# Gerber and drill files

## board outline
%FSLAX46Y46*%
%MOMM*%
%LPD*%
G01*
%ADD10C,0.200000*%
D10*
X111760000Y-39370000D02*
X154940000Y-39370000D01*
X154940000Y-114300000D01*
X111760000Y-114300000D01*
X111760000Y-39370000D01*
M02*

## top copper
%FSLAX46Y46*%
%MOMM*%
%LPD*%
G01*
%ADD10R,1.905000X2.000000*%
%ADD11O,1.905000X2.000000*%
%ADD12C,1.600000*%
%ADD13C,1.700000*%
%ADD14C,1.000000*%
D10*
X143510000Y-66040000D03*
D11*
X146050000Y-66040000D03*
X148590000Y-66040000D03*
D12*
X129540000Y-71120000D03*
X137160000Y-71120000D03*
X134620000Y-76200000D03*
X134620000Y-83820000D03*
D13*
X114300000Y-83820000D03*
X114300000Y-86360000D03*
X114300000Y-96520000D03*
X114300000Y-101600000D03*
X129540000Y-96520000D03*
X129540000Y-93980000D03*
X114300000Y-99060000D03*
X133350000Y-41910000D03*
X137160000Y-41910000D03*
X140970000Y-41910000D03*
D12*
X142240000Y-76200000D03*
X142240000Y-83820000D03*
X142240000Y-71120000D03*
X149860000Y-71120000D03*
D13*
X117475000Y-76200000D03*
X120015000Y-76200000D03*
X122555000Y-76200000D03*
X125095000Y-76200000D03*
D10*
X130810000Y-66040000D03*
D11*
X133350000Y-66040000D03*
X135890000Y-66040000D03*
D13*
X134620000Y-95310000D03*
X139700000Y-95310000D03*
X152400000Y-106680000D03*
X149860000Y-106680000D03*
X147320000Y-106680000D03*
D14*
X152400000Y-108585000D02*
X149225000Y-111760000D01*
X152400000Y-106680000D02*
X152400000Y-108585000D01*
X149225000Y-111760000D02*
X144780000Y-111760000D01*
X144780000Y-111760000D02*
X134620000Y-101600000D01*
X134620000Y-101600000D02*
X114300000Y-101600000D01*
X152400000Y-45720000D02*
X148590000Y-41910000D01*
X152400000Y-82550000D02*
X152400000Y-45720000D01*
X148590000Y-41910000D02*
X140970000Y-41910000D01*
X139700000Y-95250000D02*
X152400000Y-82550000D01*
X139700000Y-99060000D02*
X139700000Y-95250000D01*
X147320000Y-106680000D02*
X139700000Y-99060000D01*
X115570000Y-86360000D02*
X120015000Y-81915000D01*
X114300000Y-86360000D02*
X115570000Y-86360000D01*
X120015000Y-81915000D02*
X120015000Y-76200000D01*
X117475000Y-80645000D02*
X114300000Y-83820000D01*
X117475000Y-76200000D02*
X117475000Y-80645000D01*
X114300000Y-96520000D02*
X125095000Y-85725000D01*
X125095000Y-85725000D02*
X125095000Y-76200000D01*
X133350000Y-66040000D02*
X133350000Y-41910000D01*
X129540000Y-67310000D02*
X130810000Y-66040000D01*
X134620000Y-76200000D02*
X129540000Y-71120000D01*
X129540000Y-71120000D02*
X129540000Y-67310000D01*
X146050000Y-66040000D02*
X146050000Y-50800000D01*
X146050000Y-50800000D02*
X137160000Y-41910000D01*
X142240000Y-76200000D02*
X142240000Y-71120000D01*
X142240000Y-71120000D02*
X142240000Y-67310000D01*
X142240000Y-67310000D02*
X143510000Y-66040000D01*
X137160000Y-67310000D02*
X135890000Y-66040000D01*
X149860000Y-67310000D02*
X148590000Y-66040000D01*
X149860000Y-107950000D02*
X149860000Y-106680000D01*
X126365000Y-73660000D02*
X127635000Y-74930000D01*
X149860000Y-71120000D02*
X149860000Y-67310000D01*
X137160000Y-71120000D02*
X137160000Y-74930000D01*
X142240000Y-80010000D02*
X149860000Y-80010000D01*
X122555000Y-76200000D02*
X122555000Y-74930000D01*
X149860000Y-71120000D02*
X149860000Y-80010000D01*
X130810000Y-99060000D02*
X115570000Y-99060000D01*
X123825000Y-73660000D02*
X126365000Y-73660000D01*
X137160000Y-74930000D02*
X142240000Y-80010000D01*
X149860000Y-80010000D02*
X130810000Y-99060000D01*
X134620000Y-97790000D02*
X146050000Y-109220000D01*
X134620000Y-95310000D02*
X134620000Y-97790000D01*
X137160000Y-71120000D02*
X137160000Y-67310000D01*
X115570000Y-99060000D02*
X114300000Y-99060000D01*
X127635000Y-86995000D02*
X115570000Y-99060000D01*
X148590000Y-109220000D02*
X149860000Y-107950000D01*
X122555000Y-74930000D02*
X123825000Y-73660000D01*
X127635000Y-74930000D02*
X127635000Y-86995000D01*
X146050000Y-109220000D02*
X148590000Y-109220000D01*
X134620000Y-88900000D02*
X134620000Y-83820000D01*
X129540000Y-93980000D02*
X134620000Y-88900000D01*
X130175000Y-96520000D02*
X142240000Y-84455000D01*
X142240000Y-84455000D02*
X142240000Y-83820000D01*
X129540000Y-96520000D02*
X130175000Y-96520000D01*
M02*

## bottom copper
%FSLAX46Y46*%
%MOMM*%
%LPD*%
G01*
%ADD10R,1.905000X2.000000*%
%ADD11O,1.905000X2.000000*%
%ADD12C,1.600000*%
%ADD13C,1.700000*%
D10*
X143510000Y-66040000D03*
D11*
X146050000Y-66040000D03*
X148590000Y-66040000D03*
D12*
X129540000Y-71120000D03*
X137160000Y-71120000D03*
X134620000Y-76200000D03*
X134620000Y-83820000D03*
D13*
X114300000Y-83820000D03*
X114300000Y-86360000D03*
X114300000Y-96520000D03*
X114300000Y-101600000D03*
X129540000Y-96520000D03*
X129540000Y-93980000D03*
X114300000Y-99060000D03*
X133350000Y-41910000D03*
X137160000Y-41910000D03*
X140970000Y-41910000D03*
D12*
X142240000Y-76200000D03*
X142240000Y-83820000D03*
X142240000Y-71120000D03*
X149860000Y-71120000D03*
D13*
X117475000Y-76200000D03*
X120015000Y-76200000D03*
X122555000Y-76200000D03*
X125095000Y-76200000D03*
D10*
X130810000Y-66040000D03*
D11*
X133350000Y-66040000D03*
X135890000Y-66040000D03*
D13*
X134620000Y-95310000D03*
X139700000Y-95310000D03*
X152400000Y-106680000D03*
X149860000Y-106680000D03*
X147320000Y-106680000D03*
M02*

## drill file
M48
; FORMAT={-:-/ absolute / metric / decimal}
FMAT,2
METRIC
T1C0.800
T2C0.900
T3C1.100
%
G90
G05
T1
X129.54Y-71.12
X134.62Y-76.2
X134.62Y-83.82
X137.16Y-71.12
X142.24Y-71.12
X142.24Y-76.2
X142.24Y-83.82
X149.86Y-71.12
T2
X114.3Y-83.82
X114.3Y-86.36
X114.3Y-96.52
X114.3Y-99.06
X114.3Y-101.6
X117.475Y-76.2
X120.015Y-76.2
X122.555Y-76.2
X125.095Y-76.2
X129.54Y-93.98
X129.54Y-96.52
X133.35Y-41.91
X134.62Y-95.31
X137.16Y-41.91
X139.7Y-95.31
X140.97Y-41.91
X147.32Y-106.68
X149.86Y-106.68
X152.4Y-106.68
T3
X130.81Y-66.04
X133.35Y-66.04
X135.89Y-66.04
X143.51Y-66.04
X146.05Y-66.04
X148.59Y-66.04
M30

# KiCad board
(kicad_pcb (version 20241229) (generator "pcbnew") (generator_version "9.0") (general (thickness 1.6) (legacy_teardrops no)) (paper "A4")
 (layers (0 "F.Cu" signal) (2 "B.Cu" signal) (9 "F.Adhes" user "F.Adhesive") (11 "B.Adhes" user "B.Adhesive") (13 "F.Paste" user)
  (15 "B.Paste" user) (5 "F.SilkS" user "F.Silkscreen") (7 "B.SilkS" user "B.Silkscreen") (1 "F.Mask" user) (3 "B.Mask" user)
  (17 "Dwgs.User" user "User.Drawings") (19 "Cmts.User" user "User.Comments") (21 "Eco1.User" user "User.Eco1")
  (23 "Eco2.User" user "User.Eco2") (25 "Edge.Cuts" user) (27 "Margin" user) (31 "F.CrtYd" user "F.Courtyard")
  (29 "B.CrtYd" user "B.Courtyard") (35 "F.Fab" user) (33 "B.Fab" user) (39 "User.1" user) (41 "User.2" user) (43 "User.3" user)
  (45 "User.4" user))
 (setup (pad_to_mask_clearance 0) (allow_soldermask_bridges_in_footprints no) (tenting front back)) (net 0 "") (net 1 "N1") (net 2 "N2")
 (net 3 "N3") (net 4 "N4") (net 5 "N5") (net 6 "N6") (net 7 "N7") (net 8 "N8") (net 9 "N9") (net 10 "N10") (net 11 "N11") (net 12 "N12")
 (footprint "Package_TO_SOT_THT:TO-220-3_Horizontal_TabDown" (layer "F.Cu") (at 143.51 66.04)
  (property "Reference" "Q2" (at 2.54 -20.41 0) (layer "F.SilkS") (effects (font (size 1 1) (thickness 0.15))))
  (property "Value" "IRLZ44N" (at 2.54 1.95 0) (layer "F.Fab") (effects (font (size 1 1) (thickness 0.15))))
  (pad "1" thru_hole rect (at 0 0) (size 1.905 2) (drill 1.1) (layers "*.Cu" "*.Mask") (remove_unused_layers no) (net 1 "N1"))
  (pad "2" thru_hole oval (at 2.54 0) (size 1.905 2) (drill 1.1) (layers "*.Cu" "*.Mask") (remove_unused_layers no) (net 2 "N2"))
  (pad "3" thru_hole oval (at 5.08 0) (size 1.905 2) (drill 1.1) (layers "*.Cu" "*.Mask") (remove_unused_layers no) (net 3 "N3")))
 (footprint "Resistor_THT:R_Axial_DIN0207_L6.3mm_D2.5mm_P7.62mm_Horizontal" (layer "F.Cu") (at 129.54 71.12)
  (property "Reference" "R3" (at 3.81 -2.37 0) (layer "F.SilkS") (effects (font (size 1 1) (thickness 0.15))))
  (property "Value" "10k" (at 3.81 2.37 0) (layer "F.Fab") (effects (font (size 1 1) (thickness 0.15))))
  (pad "1" thru_hole circle (at 0 0) (size 1.6 1.6) (drill 0.8) (layers "*.Cu" "*.Mask") (remove_unused_layers no) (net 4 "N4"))
  (pad "2" thru_hole circle (at 7.62 0) (size 1.6 1.6) (drill 0.8) (layers "*.Cu" "*.Mask") (remove_unused_layers no) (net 3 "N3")))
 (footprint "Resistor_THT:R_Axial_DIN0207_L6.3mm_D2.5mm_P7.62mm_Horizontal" (layer "F.Cu") (at 134.62 76.2 -90)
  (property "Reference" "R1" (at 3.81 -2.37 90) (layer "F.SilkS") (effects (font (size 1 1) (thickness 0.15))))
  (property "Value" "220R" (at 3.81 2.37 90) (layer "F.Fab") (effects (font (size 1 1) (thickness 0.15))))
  (pad "1" thru_hole circle (at 0 0 270) (size 1.6 1.6) (drill 0.8) (layers "*.Cu" "*.Mask") (remove_unused_layers no) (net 4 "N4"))
  (pad "2" thru_hole circle (at 7.62 0 270) (size 1.6 1.6) (drill 0.8) (layers "*.Cu" "*.Mask") (remove_unused_layers no) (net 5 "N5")))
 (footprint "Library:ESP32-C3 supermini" (layer "F.Cu") (at 121.92 91.44)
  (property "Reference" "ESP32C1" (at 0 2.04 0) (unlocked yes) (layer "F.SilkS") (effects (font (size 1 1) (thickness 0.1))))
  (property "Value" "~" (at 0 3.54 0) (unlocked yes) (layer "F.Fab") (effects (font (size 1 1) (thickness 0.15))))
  (pad "0" thru_hole circle (at -7.62 -7.62) (size 1.7 1.7) (drill 0.9) (layers "*.Cu" "*.Mask") (remove_unused_layers yes)
   (keep_end_layers yes) (zone_layer_connections) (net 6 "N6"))
  (pad "1" thru_hole circle (at -7.62 -5.08) (size 1.7 1.7) (drill 0.9) (layers "*.Cu" "*.Mask") (remove_unused_layers yes)
   (keep_end_layers yes) (zone_layer_connections) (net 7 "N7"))
  (pad "3.3V" thru_hole circle (at -7.62 5.08) (size 1.7 1.7) (drill 0.9) (layers "*.Cu" "*.Mask") (remove_unused_layers yes)
   (keep_end_layers yes) (zone_layer_connections) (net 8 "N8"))
  (pad "5V" thru_hole circle (at -7.62 10.16) (size 1.7 1.7) (drill 0.9) (layers "*.Cu" "*.Mask") (remove_unused_layers yes)
   (keep_end_layers yes) (zone_layer_connections) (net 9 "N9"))
  (pad "7" thru_hole circle (at 7.62 5.08) (size 1.7 1.7) (drill 0.9) (layers "*.Cu" "*.Mask") (remove_unused_layers yes)
   (keep_end_layers yes) (zone_layer_connections) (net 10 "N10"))
  (pad "8" thru_hole circle (at 7.62 2.54) (size 1.7 1.7) (drill 0.9) (layers "*.Cu" "*.Mask") (remove_unused_layers yes)
   (keep_end_layers yes) (zone_layer_connections) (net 5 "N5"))
  (pad "GND" thru_hole circle (at -7.62 7.62) (size 1.7 1.7) (drill 0.9) (layers "*.Cu" "*.Mask") (remove_unused_layers yes)
   (keep_end_layers yes) (zone_layer_connections) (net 3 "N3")))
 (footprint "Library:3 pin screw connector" (layer "F.Cu") (at 137.16 41.91)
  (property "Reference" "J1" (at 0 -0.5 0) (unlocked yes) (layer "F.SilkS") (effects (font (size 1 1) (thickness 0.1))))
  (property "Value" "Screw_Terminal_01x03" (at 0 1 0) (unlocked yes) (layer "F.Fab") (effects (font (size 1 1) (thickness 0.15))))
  (pad "1" thru_hole circle (at -3.81 0) (size 1.7 1.7) (drill 0.9) (layers "*.Cu" "*.Mask") (remove_unused_layers yes)
   (keep_end_layers yes) (zone_layer_connections) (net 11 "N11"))
  (pad "2" thru_hole circle (at 0 0) (size 1.7 1.7) (drill 0.9) (layers "*.Cu" "*.Mask") (remove_unused_layers yes) (keep_end_layers yes)
   (zone_layer_connections) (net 2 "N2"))
  (pad "3" thru_hole circle (at 3.81 0) (size 1.7 1.7) (drill 0.9) (layers "*.Cu" "*.Mask") (remove_unused_layers yes) (keep_end_layers yes)
   (zone_layer_connections) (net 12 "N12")))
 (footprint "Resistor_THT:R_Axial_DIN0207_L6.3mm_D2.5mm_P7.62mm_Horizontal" (layer "F.Cu") (at 142.24 76.2 -90)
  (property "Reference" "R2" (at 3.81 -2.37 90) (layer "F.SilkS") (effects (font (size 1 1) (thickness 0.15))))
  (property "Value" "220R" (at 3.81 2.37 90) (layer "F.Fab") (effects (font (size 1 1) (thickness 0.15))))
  (pad "1" thru_hole circle (at 0 0 270) (size 1.6 1.6) (drill 0.8) (layers "*.Cu" "*.Mask") (remove_unused_layers no) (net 1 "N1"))
  (pad "2" thru_hole circle (at 7.62 0 270) (size 1.6 1.6) (drill 0.8) (layers "*.Cu" "*.Mask") (remove_unused_layers no) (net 10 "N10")))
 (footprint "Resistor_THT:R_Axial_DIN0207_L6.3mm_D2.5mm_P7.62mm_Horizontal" (layer "F.Cu") (at 142.24 71.12)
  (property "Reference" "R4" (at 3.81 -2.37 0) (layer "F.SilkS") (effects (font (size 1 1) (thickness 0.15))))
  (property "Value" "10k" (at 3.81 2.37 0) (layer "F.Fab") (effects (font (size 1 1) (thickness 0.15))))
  (pad "1" thru_hole circle (at 0 0) (size 1.6 1.6) (drill 0.8) (layers "*.Cu" "*.Mask") (remove_unused_layers no) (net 1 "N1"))
  (pad "2" thru_hole circle (at 7.62 0) (size 1.6 1.6) (drill 0.8) (layers "*.Cu" "*.Mask") (remove_unused_layers no) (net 3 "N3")))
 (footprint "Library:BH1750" (layer "F.Cu") (at 120.015 68.072)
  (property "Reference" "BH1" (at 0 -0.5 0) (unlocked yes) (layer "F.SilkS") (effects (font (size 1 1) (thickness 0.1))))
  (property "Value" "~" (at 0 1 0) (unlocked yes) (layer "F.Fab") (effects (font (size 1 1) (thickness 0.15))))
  (pad "1" thru_hole circle (at -2.54 8.128 90) (size 1.7 1.7) (drill 0.9) (layers "*.Cu" "*.Mask") (remove_unused_layers yes)
   (keep_end_layers yes) (zone_layer_connections) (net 6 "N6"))
  (pad "2" thru_hole circle (at 0 8.128 90) (size 1.7 1.7) (drill 0.9) (layers "*.Cu" "*.Mask") (remove_unused_layers yes)
   (keep_end_layers yes) (zone_layer_connections) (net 7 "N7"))
  (pad "3" thru_hole circle (at 2.54 8.128 90) (size 1.7 1.7) (drill 0.9) (layers "*.Cu" "*.Mask") (remove_unused_layers yes)
   (keep_end_layers yes) (zone_layer_connections) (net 3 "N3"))
  (pad "4" thru_hole circle (at 5.08 8.128 90) (size 1.7 1.7) (drill 0.9) (layers "*.Cu" "*.Mask") (remove_unused_layers yes)
   (keep_end_layers yes) (zone_layer_connections) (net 8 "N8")))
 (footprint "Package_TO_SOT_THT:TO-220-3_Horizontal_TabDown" (layer "F.Cu") (at 130.81 66.04)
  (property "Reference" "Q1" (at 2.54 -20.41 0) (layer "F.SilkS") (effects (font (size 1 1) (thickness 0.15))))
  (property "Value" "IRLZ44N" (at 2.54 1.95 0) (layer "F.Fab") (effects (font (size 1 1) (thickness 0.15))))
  (pad "1" thru_hole rect (at 0 0) (size 1.905 2) (drill 1.1) (layers "*.Cu" "*.Mask") (remove_unused_layers no) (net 4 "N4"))
  (pad "2" thru_hole oval (at 2.54 0) (size 1.905 2) (drill 1.1) (layers "*.Cu" "*.Mask") (remove_unused_layers no) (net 11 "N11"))
  (pad "3" thru_hole oval (at 5.08 0) (size 1.905 2) (drill 1.1) (layers "*.Cu" "*.Mask") (remove_unused_layers no) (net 3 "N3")))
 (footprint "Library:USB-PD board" (layer "F.Cu") (at 137.16 97.85)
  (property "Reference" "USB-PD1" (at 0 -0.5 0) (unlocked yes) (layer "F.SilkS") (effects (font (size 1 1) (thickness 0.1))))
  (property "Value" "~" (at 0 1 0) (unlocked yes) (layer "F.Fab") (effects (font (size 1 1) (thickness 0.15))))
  (pad "GND" thru_hole circle (at -2.54 -2.54) (size 1.7 1.7) (drill 0.9) (layers "*.Cu" "*.Mask") (remove_unused_layers yes)
   (keep_end_layers yes) (zone_layer_connections) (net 3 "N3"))
  (pad "VBUS" thru_hole circle (at 2.54 -2.54) (size 1.7 1.7) (drill 0.9) (layers "*.Cu" "*.Mask") (remove_unused_layers yes)
   (keep_end_layers yes) (zone_layer_connections) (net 12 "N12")))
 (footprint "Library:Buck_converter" (layer "F.Cu") (at 148.59 111.76 180)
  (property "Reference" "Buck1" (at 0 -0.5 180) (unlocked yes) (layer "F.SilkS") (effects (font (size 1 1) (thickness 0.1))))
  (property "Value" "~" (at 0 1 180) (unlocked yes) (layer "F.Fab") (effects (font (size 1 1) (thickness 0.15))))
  (pad "1" thru_hole circle (at -3.81 5.08 180) (size 1.7 1.7) (drill 0.9) (layers "*.Cu" "*.Mask") (remove_unused_layers yes)
   (keep_end_layers yes) (zone_layer_connections) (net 9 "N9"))
  (pad "2" thru_hole circle (at -1.27 5.08 180) (size 1.7 1.7) (drill 0.9) (layers "*.Cu" "*.Mask") (remove_unused_layers yes)
   (keep_end_layers yes) (zone_layer_connections) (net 3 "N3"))
  (pad "3" thru_hole circle (at 1.27 5.08 180) (size 1.7 1.7) (drill 0.9) (layers "*.Cu" "*.Mask") (remove_unused_layers yes)
   (keep_end_layers yes) (zone_layer_connections) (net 12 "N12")))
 (gr_rect (start 111.76 39.37) (end 154.94 114.3) (stroke (width 0.2) (type solid)) (fill no) (layer "Edge.Cuts"))
 (segment (start 152.4 108.585) (end 149.225 111.76) (width 1) (layer "F.Cu") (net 9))
 (segment (start 152.4 106.68) (end 152.4 108.585) (width 1) (layer "F.Cu") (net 9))
 (segment (start 149.225 111.76) (end 144.78 111.76) (width 1) (layer "F.Cu") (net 9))
 (segment (start 144.78 111.76) (end 134.62 101.6) (width 1) (layer "F.Cu") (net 9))
 (segment (start 134.62 101.6) (end 114.3 101.6) (width 1) (layer "F.Cu") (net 9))
 (segment (start 152.4 45.72) (end 148.59 41.91) (width 1) (layer "F.Cu") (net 12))
 (segment (start 152.4 82.55) (end 152.4 45.72) (width 1) (layer "F.Cu") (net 12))
 (segment (start 148.59 41.91) (end 140.97 41.91) (width 1) (layer "F.Cu") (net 12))
 (segment (start 139.7 95.25) (end 152.4 82.55) (width 1) (layer "F.Cu") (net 12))
 (segment (start 139.7 99.06) (end 139.7 95.25) (width 1) (layer "F.Cu") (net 12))
 (segment (start 147.32 106.68) (end 139.7 99.06) (width 1) (layer "F.Cu") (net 12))
 (segment (start 115.57 86.36) (end 120.015 81.915) (width 1) (layer "F.Cu") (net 7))
 (segment (start 114.3 86.36) (end 115.57 86.36) (width 1) (layer "F.Cu") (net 7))
 (segment (start 120.015 81.915) (end 120.015 76.2) (width 1) (layer "F.Cu") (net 7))
 (segment (start 117.475 80.645) (end 114.3 83.82) (width 1) (layer "F.Cu") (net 6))
 (segment (start 117.475 76.2) (end 117.475 80.645) (width 1) (layer "F.Cu") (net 6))
 (segment (start 114.3 96.52) (end 125.095 85.725) (width 1) (layer "F.Cu") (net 8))
 (segment (start 125.095 85.725) (end 125.095 76.2) (width 1) (layer "F.Cu") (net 8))
 (segment (start 133.35 66.04) (end 133.35 41.91) (width 1) (layer "F.Cu") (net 11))
 (segment (start 129.54 67.31) (end 130.81 66.04) (width 1) (layer "F.Cu") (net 4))
 (segment (start 134.62 76.2) (end 129.54 71.12) (width 1) (layer "F.Cu") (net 4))
 (segment (start 129.54 71.12) (end 129.54 67.31) (width 1) (layer "F.Cu") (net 4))
 (segment (start 146.05 66.04) (end 146.05 50.8) (width 1) (layer "F.Cu") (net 2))
 (segment (start 146.05 50.8) (end 137.16 41.91) (width 1) (layer "F.Cu") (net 2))
 (segment (start 142.24 76.2) (end 142.24 71.12) (width 1) (layer "F.Cu") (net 1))
 (segment (start 142.24 71.12) (end 142.24 67.31) (width 1) (layer "F.Cu") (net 1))
 (segment (start 142.24 67.31) (end 143.51 66.04) (width 1) (layer "F.Cu") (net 1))
 (segment (start 137.16 67.31) (end 135.89 66.04) (width 1) (layer "F.Cu") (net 3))
 (segment (start 149.86 67.31) (end 148.59 66.04) (width 1) (layer "F.Cu") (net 3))
 (segment (start 149.86 107.95) (end 149.86 106.68) (width 1) (layer "F.Cu") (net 3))
 (segment (start 126.365 73.66) (end 127.635 74.93) (width 1) (layer "F.Cu") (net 3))
 (segment (start 149.86 71.12) (end 149.86 67.31) (width 1) (layer "F.Cu") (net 3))
 (segment (start 137.16 71.12) (end 137.16 74.93) (width 1) (layer "F.Cu") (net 3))
 (segment (start 142.24 80.01) (end 149.86 80.01) (width 1) (layer "F.Cu") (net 3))
 (segment (start 122.555 76.2) (end 122.555 74.93) (width 1) (layer "F.Cu") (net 3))
 (segment (start 149.86 71.12) (end 149.86 80.01) (width 1) (layer "F.Cu") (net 3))
 (segment (start 130.81 99.06) (end 115.57 99.06) (width 1) (layer "F.Cu") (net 3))
 (segment (start 123.825 73.66) (end 126.365 73.66) (width 1) (layer "F.Cu") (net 3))
 (segment (start 137.16 74.93) (end 142.24 80.01) (width 1) (layer "F.Cu") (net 3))
 (segment (start 149.86 80.01) (end 130.81 99.06) (width 1) (layer "F.Cu") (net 3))
 (segment (start 134.62 97.79) (end 146.05 109.22) (width 1) (layer "F.Cu") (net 3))
 (segment (start 134.62 95.31) (end 134.62 97.79) (width 1) (layer "F.Cu") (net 3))
 (segment (start 137.16 71.12) (end 137.16 67.31) (width 1) (layer "F.Cu") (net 3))
 (segment (start 115.57 99.06) (end 114.3 99.06) (width 1) (layer "F.Cu") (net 3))
 (segment (start 127.635 86.995) (end 115.57 99.06) (width 1) (layer "F.Cu") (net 3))
 (segment (start 148.59 109.22) (end 149.86 107.95) (width 1) (layer "F.Cu") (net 3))
 (segment (start 122.555 74.93) (end 123.825 73.66) (width 1) (layer "F.Cu") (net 3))
 (segment (start 127.635 74.93) (end 127.635 86.995) (width 1) (layer "F.Cu") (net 3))
 (segment (start 146.05 109.22) (end 148.59 109.22) (width 1) (layer "F.Cu") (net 3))
 (segment (start 134.62 88.9) (end 134.62 83.82) (width 1) (layer "F.Cu") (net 5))
 (segment (start 129.54 93.98) (end 134.62 88.9) (width 1) (layer "F.Cu") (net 5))
 (segment (start 130.175 96.52) (end 142.24 84.455) (width 1) (layer "F.Cu") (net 10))
 (segment (start 142.24 84.455) (end 142.24 83.82) (width 1) (layer "F.Cu") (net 10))
 (segment (start 129.54 96.52) (end 130.175 96.52) (width 1) (layer "F.Cu") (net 10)))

